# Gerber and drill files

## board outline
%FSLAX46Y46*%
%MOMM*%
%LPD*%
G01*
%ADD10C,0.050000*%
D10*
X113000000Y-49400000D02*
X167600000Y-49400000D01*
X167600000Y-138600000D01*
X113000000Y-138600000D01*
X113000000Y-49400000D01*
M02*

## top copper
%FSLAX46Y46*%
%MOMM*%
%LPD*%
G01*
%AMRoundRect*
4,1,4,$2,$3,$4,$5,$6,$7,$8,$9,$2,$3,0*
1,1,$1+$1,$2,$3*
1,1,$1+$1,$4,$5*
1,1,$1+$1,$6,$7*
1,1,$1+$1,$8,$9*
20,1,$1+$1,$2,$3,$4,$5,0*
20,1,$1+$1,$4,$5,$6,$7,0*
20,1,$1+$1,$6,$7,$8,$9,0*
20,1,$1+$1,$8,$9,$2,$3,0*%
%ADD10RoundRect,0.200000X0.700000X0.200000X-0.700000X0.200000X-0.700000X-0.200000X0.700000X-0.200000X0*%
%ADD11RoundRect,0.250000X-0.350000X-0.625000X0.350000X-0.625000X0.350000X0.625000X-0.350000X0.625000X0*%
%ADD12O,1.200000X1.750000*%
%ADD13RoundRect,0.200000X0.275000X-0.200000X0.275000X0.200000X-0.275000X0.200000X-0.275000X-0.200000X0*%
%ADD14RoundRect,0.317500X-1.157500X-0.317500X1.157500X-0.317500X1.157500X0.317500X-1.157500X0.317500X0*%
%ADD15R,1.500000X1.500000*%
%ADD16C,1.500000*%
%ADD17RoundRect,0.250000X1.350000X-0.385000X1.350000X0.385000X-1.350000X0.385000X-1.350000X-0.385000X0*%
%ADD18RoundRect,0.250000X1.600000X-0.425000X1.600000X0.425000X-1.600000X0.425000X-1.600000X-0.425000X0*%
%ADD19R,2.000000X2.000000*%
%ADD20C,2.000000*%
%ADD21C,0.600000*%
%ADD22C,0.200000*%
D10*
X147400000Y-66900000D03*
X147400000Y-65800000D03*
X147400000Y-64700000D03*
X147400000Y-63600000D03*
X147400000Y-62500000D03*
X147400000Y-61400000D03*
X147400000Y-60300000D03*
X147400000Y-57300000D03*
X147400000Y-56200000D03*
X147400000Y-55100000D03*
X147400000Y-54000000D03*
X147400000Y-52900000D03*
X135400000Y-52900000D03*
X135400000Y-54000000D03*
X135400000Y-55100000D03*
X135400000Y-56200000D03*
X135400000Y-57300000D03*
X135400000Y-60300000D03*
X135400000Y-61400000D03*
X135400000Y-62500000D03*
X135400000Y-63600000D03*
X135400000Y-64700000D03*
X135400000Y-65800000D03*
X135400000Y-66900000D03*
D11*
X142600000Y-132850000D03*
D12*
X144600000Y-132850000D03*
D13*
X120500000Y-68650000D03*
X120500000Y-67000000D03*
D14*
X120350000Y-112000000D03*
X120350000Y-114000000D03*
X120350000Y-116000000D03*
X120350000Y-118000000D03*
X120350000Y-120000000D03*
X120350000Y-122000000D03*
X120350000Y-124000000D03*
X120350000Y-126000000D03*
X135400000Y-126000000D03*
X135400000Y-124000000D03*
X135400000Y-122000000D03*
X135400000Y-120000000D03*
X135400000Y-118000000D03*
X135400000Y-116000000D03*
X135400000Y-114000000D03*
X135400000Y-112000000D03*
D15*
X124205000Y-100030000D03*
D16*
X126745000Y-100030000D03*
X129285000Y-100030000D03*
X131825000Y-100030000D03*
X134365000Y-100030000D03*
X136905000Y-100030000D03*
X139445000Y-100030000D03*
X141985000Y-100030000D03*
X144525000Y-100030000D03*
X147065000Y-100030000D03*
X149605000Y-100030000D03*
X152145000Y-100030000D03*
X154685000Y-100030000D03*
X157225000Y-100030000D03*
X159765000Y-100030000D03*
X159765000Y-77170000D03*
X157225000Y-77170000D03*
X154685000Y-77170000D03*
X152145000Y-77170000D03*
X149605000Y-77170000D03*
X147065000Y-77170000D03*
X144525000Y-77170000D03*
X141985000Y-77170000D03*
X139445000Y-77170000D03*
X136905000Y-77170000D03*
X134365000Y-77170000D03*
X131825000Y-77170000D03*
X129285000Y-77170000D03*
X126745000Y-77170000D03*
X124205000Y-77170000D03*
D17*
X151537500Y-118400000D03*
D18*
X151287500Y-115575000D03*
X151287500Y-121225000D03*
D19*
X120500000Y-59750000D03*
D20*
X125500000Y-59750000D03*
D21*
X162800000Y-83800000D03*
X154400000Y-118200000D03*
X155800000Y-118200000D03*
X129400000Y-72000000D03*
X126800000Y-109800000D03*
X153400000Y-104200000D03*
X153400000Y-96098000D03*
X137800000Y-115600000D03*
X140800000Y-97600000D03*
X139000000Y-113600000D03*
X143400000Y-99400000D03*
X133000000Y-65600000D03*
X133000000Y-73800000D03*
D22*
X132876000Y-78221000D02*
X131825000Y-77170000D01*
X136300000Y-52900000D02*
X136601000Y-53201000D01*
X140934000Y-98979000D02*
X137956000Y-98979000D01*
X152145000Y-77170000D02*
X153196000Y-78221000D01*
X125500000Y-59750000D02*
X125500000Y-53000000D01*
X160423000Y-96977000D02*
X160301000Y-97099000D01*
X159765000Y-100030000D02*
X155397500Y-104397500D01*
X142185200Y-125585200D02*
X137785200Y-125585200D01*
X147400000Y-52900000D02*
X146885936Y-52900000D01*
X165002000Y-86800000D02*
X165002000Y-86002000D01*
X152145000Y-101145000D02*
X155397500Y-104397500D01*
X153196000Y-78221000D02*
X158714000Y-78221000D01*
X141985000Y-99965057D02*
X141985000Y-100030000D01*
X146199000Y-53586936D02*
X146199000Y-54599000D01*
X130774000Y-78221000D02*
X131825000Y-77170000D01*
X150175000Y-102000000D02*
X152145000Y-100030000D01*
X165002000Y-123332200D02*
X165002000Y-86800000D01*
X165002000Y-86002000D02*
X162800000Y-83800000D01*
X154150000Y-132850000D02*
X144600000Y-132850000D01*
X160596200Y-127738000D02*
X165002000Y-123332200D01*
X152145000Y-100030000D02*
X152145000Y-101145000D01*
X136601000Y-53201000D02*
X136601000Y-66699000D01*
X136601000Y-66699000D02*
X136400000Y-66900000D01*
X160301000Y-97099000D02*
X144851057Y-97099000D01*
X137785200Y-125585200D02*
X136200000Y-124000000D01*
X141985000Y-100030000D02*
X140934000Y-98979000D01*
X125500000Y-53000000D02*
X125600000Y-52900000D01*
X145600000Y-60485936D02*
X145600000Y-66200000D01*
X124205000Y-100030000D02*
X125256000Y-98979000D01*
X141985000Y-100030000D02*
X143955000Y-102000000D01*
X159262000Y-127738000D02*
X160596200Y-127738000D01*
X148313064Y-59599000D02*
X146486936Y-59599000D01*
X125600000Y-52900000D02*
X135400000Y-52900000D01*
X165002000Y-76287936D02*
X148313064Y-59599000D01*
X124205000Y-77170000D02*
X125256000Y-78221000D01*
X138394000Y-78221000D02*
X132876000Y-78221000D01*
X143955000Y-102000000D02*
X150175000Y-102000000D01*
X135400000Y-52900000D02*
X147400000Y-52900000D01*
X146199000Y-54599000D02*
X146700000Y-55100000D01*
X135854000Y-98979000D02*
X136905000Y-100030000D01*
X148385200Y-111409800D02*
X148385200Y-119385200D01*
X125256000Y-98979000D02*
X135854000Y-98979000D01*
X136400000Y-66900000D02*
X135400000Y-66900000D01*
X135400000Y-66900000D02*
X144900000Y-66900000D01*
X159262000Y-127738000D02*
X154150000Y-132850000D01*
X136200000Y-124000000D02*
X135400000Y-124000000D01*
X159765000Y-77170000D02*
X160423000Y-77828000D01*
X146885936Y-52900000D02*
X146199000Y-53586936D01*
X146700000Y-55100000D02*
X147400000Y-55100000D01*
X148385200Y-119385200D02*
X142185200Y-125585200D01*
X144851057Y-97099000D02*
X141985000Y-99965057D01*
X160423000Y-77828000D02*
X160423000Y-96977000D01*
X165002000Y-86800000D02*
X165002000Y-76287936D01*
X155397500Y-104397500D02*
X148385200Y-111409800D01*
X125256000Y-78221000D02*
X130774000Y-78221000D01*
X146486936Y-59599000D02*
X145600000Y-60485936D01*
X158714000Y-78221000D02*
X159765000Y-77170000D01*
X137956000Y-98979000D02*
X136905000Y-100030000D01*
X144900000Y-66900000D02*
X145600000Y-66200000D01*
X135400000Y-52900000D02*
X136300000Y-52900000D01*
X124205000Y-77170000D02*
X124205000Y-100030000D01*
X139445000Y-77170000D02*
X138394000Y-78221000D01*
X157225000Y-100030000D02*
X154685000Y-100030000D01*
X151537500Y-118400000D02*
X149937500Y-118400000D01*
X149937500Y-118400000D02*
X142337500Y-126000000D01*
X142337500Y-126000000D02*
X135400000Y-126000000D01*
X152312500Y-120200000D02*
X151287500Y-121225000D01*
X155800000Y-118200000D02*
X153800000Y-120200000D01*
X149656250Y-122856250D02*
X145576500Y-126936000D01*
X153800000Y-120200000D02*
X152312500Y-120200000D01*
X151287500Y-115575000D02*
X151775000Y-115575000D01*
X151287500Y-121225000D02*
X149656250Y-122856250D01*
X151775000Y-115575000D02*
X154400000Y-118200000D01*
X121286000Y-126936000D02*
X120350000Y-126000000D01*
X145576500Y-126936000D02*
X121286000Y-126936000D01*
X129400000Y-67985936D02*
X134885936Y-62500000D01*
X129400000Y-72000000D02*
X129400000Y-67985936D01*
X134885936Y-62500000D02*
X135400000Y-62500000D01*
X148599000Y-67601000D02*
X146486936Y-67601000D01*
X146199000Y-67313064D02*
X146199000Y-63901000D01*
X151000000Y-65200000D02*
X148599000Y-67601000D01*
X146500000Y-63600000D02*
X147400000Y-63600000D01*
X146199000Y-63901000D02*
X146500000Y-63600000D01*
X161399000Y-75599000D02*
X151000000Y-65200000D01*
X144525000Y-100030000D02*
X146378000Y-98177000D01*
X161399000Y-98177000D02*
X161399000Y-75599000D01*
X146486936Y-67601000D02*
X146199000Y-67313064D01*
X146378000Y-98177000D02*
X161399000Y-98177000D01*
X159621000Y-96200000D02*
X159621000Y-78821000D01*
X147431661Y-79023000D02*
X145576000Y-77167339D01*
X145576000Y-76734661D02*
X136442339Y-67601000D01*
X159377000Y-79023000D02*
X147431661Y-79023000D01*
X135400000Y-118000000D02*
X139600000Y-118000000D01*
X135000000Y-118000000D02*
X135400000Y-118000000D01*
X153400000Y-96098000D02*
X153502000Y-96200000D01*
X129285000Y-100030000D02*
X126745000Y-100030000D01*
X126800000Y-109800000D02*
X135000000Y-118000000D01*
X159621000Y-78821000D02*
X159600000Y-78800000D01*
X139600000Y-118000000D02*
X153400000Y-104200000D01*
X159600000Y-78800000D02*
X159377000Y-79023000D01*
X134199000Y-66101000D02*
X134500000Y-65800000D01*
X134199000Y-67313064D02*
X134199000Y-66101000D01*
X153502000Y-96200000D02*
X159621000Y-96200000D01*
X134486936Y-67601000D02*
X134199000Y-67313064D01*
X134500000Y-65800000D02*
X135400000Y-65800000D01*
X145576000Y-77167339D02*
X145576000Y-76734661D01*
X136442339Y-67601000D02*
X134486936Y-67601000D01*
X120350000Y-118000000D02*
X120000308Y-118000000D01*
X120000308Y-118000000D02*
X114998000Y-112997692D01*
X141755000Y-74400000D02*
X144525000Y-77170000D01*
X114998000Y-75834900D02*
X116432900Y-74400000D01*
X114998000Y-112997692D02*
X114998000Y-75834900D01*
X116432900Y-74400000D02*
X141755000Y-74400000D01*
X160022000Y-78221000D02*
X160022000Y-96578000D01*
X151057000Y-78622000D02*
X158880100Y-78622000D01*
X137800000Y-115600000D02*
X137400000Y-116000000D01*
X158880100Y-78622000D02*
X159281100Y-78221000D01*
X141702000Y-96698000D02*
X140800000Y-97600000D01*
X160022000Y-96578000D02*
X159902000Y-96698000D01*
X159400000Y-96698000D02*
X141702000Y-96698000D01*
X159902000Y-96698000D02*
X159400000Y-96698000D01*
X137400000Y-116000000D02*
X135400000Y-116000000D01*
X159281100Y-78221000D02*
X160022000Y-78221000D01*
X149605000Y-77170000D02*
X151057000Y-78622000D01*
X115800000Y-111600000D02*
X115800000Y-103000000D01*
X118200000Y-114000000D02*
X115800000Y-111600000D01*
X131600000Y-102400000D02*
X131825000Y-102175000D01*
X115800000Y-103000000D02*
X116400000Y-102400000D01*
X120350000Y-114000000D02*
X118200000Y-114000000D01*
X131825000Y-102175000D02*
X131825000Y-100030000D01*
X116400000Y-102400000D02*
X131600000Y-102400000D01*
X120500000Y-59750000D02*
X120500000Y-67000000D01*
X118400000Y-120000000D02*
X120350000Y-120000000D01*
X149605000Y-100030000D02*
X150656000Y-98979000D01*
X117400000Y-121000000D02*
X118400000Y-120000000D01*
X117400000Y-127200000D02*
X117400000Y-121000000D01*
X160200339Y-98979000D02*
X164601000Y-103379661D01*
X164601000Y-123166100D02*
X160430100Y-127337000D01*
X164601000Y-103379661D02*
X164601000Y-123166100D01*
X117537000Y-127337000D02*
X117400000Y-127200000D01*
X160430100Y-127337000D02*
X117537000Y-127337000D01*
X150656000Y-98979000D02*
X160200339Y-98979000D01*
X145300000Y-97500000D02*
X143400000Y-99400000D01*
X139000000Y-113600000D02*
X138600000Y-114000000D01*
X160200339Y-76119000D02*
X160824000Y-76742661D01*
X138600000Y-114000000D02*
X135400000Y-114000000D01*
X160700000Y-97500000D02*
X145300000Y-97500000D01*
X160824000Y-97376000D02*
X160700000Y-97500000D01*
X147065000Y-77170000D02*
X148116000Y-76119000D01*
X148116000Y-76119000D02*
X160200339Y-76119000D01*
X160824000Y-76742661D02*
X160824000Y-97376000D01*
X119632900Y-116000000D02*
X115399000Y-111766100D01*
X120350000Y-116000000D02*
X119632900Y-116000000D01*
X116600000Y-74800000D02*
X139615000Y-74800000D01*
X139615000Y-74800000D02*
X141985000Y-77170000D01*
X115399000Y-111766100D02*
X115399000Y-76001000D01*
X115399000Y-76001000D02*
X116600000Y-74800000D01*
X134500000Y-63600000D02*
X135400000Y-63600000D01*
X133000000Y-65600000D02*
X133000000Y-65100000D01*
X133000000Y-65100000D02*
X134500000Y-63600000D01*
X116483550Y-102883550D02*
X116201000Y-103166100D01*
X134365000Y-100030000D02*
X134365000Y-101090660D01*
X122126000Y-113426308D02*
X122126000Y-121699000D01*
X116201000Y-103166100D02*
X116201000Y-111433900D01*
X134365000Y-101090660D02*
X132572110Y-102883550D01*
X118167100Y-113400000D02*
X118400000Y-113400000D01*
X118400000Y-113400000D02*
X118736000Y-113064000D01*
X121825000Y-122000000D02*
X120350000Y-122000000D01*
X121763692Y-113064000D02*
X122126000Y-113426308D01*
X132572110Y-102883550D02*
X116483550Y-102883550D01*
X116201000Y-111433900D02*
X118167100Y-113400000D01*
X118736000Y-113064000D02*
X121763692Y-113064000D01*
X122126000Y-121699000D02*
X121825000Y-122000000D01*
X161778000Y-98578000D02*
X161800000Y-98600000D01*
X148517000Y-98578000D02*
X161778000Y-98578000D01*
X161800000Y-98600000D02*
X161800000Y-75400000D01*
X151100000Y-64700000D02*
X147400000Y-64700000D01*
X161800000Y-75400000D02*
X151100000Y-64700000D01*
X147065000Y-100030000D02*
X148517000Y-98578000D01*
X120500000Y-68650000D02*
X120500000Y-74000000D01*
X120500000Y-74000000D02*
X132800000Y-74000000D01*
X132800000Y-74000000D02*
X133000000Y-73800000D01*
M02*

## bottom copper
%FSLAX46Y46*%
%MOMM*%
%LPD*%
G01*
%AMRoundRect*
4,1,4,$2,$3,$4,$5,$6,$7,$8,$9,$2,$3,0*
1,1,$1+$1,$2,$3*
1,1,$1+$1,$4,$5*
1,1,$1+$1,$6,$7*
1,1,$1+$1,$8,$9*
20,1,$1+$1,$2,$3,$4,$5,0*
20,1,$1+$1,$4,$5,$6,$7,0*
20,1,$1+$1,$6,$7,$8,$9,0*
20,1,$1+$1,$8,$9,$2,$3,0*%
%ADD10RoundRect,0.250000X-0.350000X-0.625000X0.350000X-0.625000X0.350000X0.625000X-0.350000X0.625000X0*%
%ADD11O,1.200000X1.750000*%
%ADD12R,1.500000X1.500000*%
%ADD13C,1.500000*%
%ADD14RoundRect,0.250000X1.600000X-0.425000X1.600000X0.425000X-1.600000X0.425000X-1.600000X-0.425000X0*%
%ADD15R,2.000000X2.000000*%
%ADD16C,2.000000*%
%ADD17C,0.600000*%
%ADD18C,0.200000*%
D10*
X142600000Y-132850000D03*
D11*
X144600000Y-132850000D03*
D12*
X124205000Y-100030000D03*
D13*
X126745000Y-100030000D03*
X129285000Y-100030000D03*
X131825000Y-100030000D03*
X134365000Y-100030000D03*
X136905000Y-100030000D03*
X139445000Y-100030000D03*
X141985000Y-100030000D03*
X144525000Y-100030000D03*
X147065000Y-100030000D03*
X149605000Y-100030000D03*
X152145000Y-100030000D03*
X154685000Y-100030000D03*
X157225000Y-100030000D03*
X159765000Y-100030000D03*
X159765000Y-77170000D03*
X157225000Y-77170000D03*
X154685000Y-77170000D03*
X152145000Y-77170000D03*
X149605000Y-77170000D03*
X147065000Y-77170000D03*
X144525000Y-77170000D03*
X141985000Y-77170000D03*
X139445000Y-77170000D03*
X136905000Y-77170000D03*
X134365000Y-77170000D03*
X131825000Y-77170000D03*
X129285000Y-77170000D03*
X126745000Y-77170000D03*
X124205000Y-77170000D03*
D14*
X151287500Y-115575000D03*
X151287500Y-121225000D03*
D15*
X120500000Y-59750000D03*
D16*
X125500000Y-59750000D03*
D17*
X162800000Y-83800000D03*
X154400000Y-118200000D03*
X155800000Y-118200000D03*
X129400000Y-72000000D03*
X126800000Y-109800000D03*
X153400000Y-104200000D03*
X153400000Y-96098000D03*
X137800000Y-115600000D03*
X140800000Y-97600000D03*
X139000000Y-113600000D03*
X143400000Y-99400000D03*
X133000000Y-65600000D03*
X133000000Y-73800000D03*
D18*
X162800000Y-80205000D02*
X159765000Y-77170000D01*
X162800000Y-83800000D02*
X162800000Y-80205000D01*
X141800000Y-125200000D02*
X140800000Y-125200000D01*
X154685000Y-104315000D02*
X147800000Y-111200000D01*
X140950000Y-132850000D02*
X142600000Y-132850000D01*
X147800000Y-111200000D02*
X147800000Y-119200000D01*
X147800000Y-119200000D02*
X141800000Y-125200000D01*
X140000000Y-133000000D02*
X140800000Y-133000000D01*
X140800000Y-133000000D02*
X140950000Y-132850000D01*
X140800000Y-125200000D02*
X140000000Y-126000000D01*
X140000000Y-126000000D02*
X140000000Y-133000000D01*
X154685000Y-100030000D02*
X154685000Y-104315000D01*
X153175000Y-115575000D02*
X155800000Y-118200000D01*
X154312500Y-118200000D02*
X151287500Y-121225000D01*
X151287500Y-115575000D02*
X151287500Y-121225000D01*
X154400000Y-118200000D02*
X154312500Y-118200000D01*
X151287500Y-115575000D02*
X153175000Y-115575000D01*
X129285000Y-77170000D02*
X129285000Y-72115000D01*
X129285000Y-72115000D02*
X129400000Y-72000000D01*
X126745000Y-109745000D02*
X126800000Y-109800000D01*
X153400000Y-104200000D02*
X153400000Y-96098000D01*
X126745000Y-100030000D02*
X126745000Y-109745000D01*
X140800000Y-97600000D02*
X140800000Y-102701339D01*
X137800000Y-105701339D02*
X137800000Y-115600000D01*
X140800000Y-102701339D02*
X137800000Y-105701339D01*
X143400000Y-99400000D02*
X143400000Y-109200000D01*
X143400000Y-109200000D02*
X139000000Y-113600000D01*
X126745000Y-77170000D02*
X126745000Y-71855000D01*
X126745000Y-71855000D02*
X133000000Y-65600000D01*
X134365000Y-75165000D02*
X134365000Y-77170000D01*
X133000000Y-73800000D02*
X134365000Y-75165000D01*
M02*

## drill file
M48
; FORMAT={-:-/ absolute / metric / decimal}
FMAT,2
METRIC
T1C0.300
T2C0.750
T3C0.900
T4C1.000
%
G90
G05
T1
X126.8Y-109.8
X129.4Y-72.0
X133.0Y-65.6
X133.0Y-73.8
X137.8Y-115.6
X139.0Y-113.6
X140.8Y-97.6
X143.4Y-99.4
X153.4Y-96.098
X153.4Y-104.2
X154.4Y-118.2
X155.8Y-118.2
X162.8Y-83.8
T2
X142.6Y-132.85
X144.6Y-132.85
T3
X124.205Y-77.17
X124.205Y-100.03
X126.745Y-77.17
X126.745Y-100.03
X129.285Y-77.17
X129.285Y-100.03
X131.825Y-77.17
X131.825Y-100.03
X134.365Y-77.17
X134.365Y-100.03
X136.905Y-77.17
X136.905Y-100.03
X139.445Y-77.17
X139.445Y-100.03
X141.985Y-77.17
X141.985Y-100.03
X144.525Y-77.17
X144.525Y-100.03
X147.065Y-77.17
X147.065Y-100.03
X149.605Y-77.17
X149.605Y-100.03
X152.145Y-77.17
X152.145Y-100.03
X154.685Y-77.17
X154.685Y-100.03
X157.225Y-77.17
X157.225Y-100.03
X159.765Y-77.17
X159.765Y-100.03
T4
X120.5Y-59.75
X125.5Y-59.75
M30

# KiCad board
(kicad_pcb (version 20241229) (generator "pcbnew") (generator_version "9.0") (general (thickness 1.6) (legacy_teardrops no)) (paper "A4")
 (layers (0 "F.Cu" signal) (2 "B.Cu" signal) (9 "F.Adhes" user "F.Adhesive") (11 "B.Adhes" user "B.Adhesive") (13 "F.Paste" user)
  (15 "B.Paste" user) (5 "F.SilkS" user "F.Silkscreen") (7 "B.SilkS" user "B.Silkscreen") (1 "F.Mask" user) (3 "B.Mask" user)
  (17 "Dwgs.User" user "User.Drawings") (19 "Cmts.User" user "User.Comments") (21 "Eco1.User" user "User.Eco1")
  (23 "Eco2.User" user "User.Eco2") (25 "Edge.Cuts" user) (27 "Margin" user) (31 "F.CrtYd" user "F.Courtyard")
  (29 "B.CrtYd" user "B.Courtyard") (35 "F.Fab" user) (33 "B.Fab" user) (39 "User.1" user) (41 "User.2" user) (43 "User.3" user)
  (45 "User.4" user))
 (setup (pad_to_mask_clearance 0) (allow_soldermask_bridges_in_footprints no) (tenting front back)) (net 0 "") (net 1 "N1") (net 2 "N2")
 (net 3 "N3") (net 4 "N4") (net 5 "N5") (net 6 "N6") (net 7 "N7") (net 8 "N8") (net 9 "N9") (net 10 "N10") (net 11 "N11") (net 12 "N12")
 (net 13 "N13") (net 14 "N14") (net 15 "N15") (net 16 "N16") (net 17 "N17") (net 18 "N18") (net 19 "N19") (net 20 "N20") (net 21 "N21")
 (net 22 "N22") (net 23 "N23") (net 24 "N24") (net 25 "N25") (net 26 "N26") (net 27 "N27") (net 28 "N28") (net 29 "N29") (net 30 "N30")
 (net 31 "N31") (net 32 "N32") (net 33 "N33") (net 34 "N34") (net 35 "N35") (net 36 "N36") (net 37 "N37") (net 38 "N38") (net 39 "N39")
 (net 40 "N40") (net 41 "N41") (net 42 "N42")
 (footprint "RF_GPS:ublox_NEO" (layer "F.Cu") (at 141.4 59.9 180)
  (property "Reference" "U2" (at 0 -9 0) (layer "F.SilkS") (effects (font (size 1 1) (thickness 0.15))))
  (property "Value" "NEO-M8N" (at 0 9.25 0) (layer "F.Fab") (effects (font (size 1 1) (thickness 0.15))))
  (pad "1" smd roundrect (at -6 -7 180) (size 1.8 0.8) (layers "F.Cu" "F.Mask" "F.Paste") (roundrect_rratio 0.25) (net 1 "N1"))
  (pad "2" smd roundrect (at -6 -5.9 180) (size 1.8 0.8) (layers "F.Cu" "F.Mask" "F.Paste") (roundrect_rratio 0.25) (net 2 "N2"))
  (pad "3" smd roundrect (at -6 -4.8 180) (size 1.8 0.8) (layers "F.Cu" "F.Mask" "F.Paste") (roundrect_rratio 0.25) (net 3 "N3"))
  (pad "4" smd roundrect (at -6 -3.7 180) (size 1.8 0.8) (layers "F.Cu" "F.Mask" "F.Paste") (roundrect_rratio 0.25) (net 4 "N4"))
  (pad "5" smd roundrect (at -6 -2.6 180) (size 1.8 0.8) (layers "F.Cu" "F.Mask" "F.Paste") (roundrect_rratio 0.25) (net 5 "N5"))
  (pad "6" smd roundrect (at -6 -1.5 180) (size 1.8 0.8) (layers "F.Cu" "F.Mask" "F.Paste") (roundrect_rratio 0.25) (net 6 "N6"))
  (pad "7" smd roundrect (at -6 -0.4 180) (size 1.8 0.8) (layers "F.Cu" "F.Mask" "F.Paste") (roundrect_rratio 0.25) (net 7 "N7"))
  (pad "8" smd roundrect (at -6 2.6 180) (size 1.8 0.8) (layers "F.Cu" "F.Mask" "F.Paste") (roundrect_rratio 0.25) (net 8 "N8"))
  (pad "9" smd roundrect (at -6 3.7 180) (size 1.8 0.8) (layers "F.Cu" "F.Mask" "F.Paste") (roundrect_rratio 0.25) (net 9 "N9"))
  (pad "10" smd roundrect (at -6 4.8 180) (size 1.8 0.8) (layers "F.Cu" "F.Mask" "F.Paste") (roundrect_rratio 0.25) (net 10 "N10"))
  (pad "11" smd roundrect (at -6 5.9 180) (size 1.8 0.8) (layers "F.Cu" "F.Mask" "F.Paste") (roundrect_rratio 0.25) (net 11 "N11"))
  (pad "12" smd roundrect (at -6 7 180) (size 1.8 0.8) (layers "F.Cu" "F.Mask" "F.Paste") (roundrect_rratio 0.25) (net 10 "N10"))
  (pad "13" smd roundrect (at 6 7 180) (size 1.8 0.8) (layers "F.Cu" "F.Mask" "F.Paste") (roundrect_rratio 0.25) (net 10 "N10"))
  (pad "14" smd roundrect (at 6 5.9 180) (size 1.8 0.8) (layers "F.Cu" "F.Mask" "F.Paste") (roundrect_rratio 0.25) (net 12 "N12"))
  (pad "15" smd roundrect (at 6 4.8 180) (size 1.8 0.8) (layers "F.Cu" "F.Mask" "F.Paste") (roundrect_rratio 0.25) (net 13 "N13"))
  (pad "16" smd roundrect (at 6 3.7 180) (size 1.8 0.8) (layers "F.Cu" "F.Mask" "F.Paste") (roundrect_rratio 0.25) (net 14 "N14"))
  (pad "17" smd roundrect (at 6 2.6 180) (size 1.8 0.8) (layers "F.Cu" "F.Mask" "F.Paste") (roundrect_rratio 0.25) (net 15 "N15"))
  (pad "18" smd roundrect (at 6 -0.4 180) (size 1.8 0.8) (layers "F.Cu" "F.Mask" "F.Paste") (roundrect_rratio 0.25) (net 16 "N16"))
  (pad "19" smd roundrect (at 6 -1.5 180) (size 1.8 0.8) (layers "F.Cu" "F.Mask" "F.Paste") (roundrect_rratio 0.25) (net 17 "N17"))
  (pad "20" smd roundrect (at 6 -2.6 180) (size 1.8 0.8) (layers "F.Cu" "F.Mask" "F.Paste") (roundrect_rratio 0.25) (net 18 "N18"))
  (pad "21" smd roundrect (at 6 -3.7 180) (size 1.8 0.8) (layers "F.Cu" "F.Mask" "F.Paste") (roundrect_rratio 0.25) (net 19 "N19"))
  (pad "22" smd roundrect (at 6 -4.8 180) (size 1.8 0.8) (layers "F.Cu" "F.Mask" "F.Paste") (roundrect_rratio 0.25) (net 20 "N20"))
  (pad "23" smd roundrect (at 6 -5.9 180) (size 1.8 0.8) (layers "F.Cu" "F.Mask" "F.Paste") (roundrect_rratio 0.25) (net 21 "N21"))
  (pad "24" smd roundrect (at 6 -7 180) (size 1.8 0.8) (layers "F.Cu" "F.Mask" "F.Paste") (roundrect_rratio 0.25) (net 10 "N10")))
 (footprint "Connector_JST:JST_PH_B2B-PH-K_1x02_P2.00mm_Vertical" (layer "F.Cu") (at 142.6 132.85)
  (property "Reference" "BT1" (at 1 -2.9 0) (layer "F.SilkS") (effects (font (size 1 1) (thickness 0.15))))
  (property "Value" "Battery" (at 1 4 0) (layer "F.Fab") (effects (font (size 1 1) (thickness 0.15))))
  (pad "1" thru_hole roundrect (at 0 0) (size 1.2 1.75) (drill 0.75) (layers "*.Cu" "*.Mask") (remove_unused_layers no)
   (roundrect_rratio 0.208333) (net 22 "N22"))
  (pad "2" thru_hole oval (at 2 0) (size 1.2 1.75) (drill 0.75) (layers "*.Cu" "*.Mask") (remove_unused_layers no) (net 10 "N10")))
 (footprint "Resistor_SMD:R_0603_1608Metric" (layer "F.Cu") (at 120.5 67.825 90)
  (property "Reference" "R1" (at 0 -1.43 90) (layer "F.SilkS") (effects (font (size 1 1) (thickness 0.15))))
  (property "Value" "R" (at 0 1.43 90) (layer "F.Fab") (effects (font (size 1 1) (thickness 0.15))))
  (pad "1" smd roundrect (at -0.825 0 90) (size 0.8 0.95) (layers "F.Cu" "F.Mask" "F.Paste") (roundrect_rratio 0.25) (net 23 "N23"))
  (pad "2" smd roundrect (at 0.825 0 90) (size 0.8 0.95) (layers "F.Cu" "F.Mask" "F.Paste") (roundrect_rratio 0.25) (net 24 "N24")))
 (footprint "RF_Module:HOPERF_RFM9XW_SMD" (layer "F.Cu") (at 127.875 119)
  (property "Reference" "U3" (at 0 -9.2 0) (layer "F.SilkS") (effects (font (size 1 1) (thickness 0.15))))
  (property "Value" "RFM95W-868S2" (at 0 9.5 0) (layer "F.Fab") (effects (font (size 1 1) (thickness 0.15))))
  (pad "1" smd roundrect (at -7.525 -7) (size 2.95 1.27) (layers "F.Cu" "F.Mask" "F.Paste") (roundrect_rratio 0.25) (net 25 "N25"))
  (pad "2" smd roundrect (at -7.525 -5) (size 2.95 1.27) (layers "F.Cu" "F.Mask" "F.Paste") (roundrect_rratio 0.25) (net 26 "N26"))
  (pad "3" smd roundrect (at -7.525 -3) (size 2.95 1.27) (layers "F.Cu" "F.Mask" "F.Paste") (roundrect_rratio 0.25) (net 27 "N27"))
  (pad "4" smd roundrect (at -7.525 -1) (size 2.95 1.27) (layers "F.Cu" "F.Mask" "F.Paste") (roundrect_rratio 0.25) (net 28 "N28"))
  (pad "5" smd roundrect (at -7.525 1) (size 2.95 1.27) (layers "F.Cu" "F.Mask" "F.Paste") (roundrect_rratio 0.25) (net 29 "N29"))
  (pad "6" smd roundrect (at -7.525 3) (size 2.95 1.27) (layers "F.Cu" "F.Mask" "F.Paste") (roundrect_rratio 0.25) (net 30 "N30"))
  (pad "7" smd roundrect (at -7.525 5) (size 2.95 1.27) (layers "F.Cu" "F.Mask" "F.Paste") (roundrect_rratio 0.25) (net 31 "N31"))
  (pad "8" smd roundrect (at -7.525 7) (size 2.95 1.27) (layers "F.Cu" "F.Mask" "F.Paste") (roundrect_rratio 0.25) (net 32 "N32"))
  (pad "9" smd roundrect (at 7.525 7) (size 2.95 1.27) (layers "F.Cu" "F.Mask" "F.Paste") (roundrect_rratio 0.25) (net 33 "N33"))
  (pad "10" smd roundrect (at 7.525 5) (size 2.95 1.27) (layers "F.Cu" "F.Mask" "F.Paste") (roundrect_rratio 0.25) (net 10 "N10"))
  (pad "11" smd roundrect (at 7.525 3) (size 2.95 1.27) (layers "F.Cu" "F.Mask" "F.Paste") (roundrect_rratio 0.25) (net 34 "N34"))
  (pad "12" smd roundrect (at 7.525 1) (size 2.95 1.27) (layers "F.Cu" "F.Mask" "F.Paste") (roundrect_rratio 0.25) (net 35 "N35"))
  (pad "13" smd roundrect (at 7.525 -1) (size 2.95 1.27) (layers "F.Cu" "F.Mask" "F.Paste") (roundrect_rratio 0.25) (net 21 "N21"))
  (pad "14" smd roundrect (at 7.525 -3) (size 2.95 1.27) (layers "F.Cu" "F.Mask" "F.Paste") (roundrect_rratio 0.25) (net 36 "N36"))
  (pad "15" smd roundrect (at 7.525 -5) (size 2.95 1.27) (layers "F.Cu" "F.Mask" "F.Paste") (roundrect_rratio 0.25) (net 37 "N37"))
  (pad "16" smd roundrect (at 7.525 -7) (size 2.95 1.27) (layers "F.Cu" "F.Mask" "F.Paste") (roundrect_rratio 0.25) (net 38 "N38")))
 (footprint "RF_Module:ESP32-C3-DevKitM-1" (layer "F.Cu") (at 124.205 100.03 90)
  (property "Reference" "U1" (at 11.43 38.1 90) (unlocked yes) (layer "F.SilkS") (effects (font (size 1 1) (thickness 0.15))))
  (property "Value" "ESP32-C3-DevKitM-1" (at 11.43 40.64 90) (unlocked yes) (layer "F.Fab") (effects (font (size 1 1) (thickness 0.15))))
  (pad "1" thru_hole rect (at 0 0 90) (size 1.5 1.5) (drill 0.9) (layers "*.Cu" "*.Mask") (remove_unused_layers yes) (keep_end_layers yes)
   (zone_layer_connections) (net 10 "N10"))
  (pad "2" thru_hole circle (at 0 2.54 90) (size 1.5 1.5) (drill 0.9) (layers "*.Cu" "*.Mask") (remove_unused_layers yes)
   (keep_end_layers yes) (zone_layer_connections) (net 21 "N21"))
  (pad "3" thru_hole circle (at 0 5.08 90) (size 1.5 1.5) (drill 0.9) (layers "*.Cu" "*.Mask") (remove_unused_layers yes)
   (keep_end_layers yes) (zone_layer_connections) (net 21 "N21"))
  (pad "4" thru_hole circle (at 0 7.62 90) (size 1.5 1.5) (drill 0.9) (layers "*.Cu" "*.Mask") (remove_unused_layers yes)
   (keep_end_layers yes) (zone_layer_connections) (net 26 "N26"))
  (pad "5" thru_hole circle (at 0 10.16 90) (size 1.5 1.5) (drill 0.9) (layers "*.Cu" "*.Mask") (remove_unused_layers yes)
   (keep_end_layers yes) (zone_layer_connections) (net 30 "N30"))
  (pad "6" thru_hole circle (at 0 12.7 90) (size 1.5 1.5) (drill 0.9) (layers "*.Cu" "*.Mask") (remove_unused_layers yes)
   (keep_end_layers yes) (zone_layer_connections) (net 10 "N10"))
  (pad "7" thru_hole circle (at 0 15.24 90) (size 1.5 1.5) (drill 0.9) (layers "*.Cu" "*.Mask") (remove_unused_layers yes)
   (keep_end_layers yes) (zone_layer_connections) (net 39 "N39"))
  (pad "8" thru_hole circle (at 0 17.78 90) (size 1.5 1.5) (drill 0.9) (layers "*.Cu" "*.Mask") (remove_unused_layers yes)
   (keep_end_layers yes) (zone_layer_connections) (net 10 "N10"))
  (pad "9" thru_hole circle (at 0 20.32 90) (size 1.5 1.5) (drill 0.9) (layers "*.Cu" "*.Mask") (remove_unused_layers yes)
   (keep_end_layers yes) (zone_layer_connections) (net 4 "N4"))
  (pad "10" thru_hole circle (at 0 22.86 90) (size 1.5 1.5) (drill 0.9) (layers "*.Cu" "*.Mask") (remove_unused_layers yes)
   (keep_end_layers yes) (zone_layer_connections) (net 3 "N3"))
  (pad "11" thru_hole circle (at 0 25.4 90) (size 1.5 1.5) (drill 0.9) (layers "*.Cu" "*.Mask") (remove_unused_layers yes)
   (keep_end_layers yes) (zone_layer_connections) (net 29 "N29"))
  (pad "12" thru_hole circle (at 0 27.94 90) (size 1.5 1.5) (drill 0.9) (layers "*.Cu" "*.Mask") (remove_unused_layers yes)
   (keep_end_layers yes) (zone_layer_connections) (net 10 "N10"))
  (pad "13" thru_hole circle (at 0 30.48 90) (size 1.5 1.5) (drill 0.9) (layers "*.Cu" "*.Mask") (remove_unused_layers yes)
   (keep_end_layers yes) (zone_layer_connections) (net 22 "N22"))
  (pad "14" thru_hole circle (at 0 33.02 90) (size 1.5 1.5) (drill 0.9) (layers "*.Cu" "*.Mask") (remove_unused_layers yes)
   (keep_end_layers yes) (zone_layer_connections) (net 22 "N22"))
  (pad "15" thru_hole circle (at 0 35.56 90) (size 1.5 1.5) (drill 0.9) (layers "*.Cu" "*.Mask") (remove_unused_layers yes)
   (keep_end_layers yes) (zone_layer_connections) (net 10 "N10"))
  (pad "16" thru_hole circle (at 22.86 35.56 90) (size 1.5 1.5) (drill 0.9) (layers "*.Cu" "*.Mask") (remove_unused_layers yes)
   (keep_end_layers yes) (zone_layer_connections) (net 10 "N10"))
  (pad "17" thru_hole circle (at 22.86 33.02 90) (size 1.5 1.5) (drill 0.9) (layers "*.Cu" "*.Mask") (remove_unused_layers yes)
   (keep_end_layers yes) (zone_layer_connections) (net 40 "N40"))
  (pad "18" thru_hole circle (at 22.86 30.48 90) (size 1.5 1.5) (drill 0.9) (layers "*.Cu" "*.Mask") (remove_unused_layers yes)
   (keep_end_layers yes) (zone_layer_connections) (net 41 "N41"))
  (pad "19" thru_hole circle (at 22.86 27.94 90) (size 1.5 1.5) (drill 0.9) (layers "*.Cu" "*.Mask") (remove_unused_layers yes)
   (keep_end_layers yes) (zone_layer_connections) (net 10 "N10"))
  (pad "20" thru_hole circle (at 22.86 25.4 90) (size 1.5 1.5) (drill 0.9) (layers "*.Cu" "*.Mask") (remove_unused_layers yes)
   (keep_end_layers yes) (zone_layer_connections) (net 36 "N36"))
  (pad "21" thru_hole circle (at 22.86 22.86 90) (size 1.5 1.5) (drill 0.9) (layers "*.Cu" "*.Mask") (remove_unused_layers yes)
   (keep_end_layers yes) (zone_layer_connections) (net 37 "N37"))
  (pad "22" thru_hole circle (at 22.86 20.32 90) (size 1.5 1.5) (drill 0.9) (layers "*.Cu" "*.Mask") (remove_unused_layers yes)
   (keep_end_layers yes) (zone_layer_connections) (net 28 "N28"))
  (pad "23" thru_hole circle (at 22.86 17.78 90) (size 1.5 1.5) (drill 0.9) (layers "*.Cu" "*.Mask") (remove_unused_layers yes)
   (keep_end_layers yes) (zone_layer_connections) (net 27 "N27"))
  (pad "24" thru_hole circle (at 22.86 15.24 90) (size 1.5 1.5) (drill 0.9) (layers "*.Cu" "*.Mask") (remove_unused_layers yes)
   (keep_end_layers yes) (zone_layer_connections) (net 10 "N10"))
  (pad "25" thru_hole circle (at 22.86 12.7 90) (size 1.5 1.5) (drill 0.9) (layers "*.Cu" "*.Mask") (remove_unused_layers yes)
   (keep_end_layers yes) (zone_layer_connections) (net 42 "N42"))
  (pad "26" thru_hole circle (at 22.86 10.16 90) (size 1.5 1.5) (drill 0.9) (layers "*.Cu" "*.Mask") (remove_unused_layers yes)
   (keep_end_layers yes) (zone_layer_connections) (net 23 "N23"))
  (pad "27" thru_hole circle (at 22.86 7.62 90) (size 1.5 1.5) (drill 0.9) (layers "*.Cu" "*.Mask") (remove_unused_layers yes)
   (keep_end_layers yes) (zone_layer_connections) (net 10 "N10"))
  (pad "28" thru_hole circle (at 22.86 5.08 90) (size 1.5 1.5) (drill 0.9) (layers "*.Cu" "*.Mask") (remove_unused_layers yes)
   (keep_end_layers yes) (zone_layer_connections) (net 18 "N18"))
  (pad "29" thru_hole circle (at 22.86 2.54 90) (size 1.5 1.5) (drill 0.9) (layers "*.Cu" "*.Mask") (remove_unused_layers yes)
   (keep_end_layers yes) (zone_layer_connections) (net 19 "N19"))
  (pad "30" thru_hole circle (at 22.86 0 90) (size 1.5 1.5) (drill 0.9) (layers "*.Cu" "*.Mask") (remove_unused_layers yes)
   (keep_end_layers yes) (zone_layer_connections) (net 10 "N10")))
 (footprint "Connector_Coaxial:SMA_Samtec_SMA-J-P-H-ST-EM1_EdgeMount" (layer "F.Cu") (at 151.5375 118.4)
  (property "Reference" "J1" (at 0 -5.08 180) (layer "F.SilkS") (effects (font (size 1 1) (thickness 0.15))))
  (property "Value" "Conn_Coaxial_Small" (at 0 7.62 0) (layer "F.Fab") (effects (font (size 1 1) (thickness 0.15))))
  (pad "1" smd roundrect (at 0 0 90) (size 1.27 3.2) (layers "F.Cu" "F.Mask") (roundrect_rratio 0.1968503937) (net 33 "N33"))
  (pad "2" smd roundrect (at -0.25 -2.825 90) (size 1.35 3.7) (layers "F.Cu" "F.Mask") (roundrect_rratio 0.1851851852) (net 32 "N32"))
  (pad "2" smd roundrect (at -0.25 -2.825 90) (size 1.35 3.7) (layers "B.Cu" "B.Mask") (roundrect_rratio 0.1851851852) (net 32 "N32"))
  (pad "2" smd roundrect (at -0.25 2.825 90) (size 1.35 3.7) (layers "F.Cu" "F.Mask") (roundrect_rratio 0.1851851852) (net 32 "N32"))
  (pad "2" smd roundrect (at -0.25 2.825 90) (size 1.35 3.7) (layers "B.Cu" "B.Mask") (roundrect_rratio 0.1851851852) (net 32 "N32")))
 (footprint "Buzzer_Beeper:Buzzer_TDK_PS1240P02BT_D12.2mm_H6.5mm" (layer "F.Cu") (at 120.5 59.75)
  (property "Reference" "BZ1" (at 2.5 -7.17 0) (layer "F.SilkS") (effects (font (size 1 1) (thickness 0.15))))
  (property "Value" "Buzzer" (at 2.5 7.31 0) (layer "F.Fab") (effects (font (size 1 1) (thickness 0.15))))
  (pad "1" thru_hole rect (at 0 0) (size 2 2) (drill 1) (layers "*.Cu" "*.Mask") (remove_unused_layers no) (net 24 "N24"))
  (pad "2" thru_hole circle (at 5 0) (size 2 2) (drill 1) (layers "*.Cu" "*.Mask") (remove_unused_layers no) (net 10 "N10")))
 (gr_rect (start 113 49.4) (end 167.6 138.6) (stroke (width 0.05) (type default)) (fill no) (layer "Edge.Cuts"))
 (segment (start 132.876 78.221) (end 131.825 77.17) (width 0.2) (layer "F.Cu") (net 10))
 (segment (start 136.3 52.9) (end 136.601 53.201) (width 0.2) (layer "F.Cu") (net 10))
 (segment (start 140.934 98.979) (end 137.956 98.979) (width 0.2) (layer "F.Cu") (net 10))
 (segment (start 152.145 77.17) (end 153.196 78.221) (width 0.2) (layer "F.Cu") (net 10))
 (segment (start 125.5 59.75) (end 125.5 53) (width 0.2) (layer "F.Cu") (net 10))
 (segment (start 160.423 96.977) (end 160.301 97.099) (width 0.2) (layer "F.Cu") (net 10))
 (segment (start 159.765 100.03) (end 155.3975 104.3975) (width 0.2) (layer "F.Cu") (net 10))
 (segment (start 142.1852 125.5852) (end 137.7852 125.5852) (width 0.2) (layer "F.Cu") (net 10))
 (segment (start 147.4 52.9) (end 146.885936 52.9) (width 0.2) (layer "F.Cu") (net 10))
 (segment (start 165.002 86.8) (end 165.002 86.002) (width 0.2) (layer "F.Cu") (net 10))
 (segment (start 152.145 101.145) (end 155.3975 104.3975) (width 0.2) (layer "F.Cu") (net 10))
 (segment (start 153.196 78.221) (end 158.714 78.221) (width 0.2) (layer "F.Cu") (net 10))
 (segment (start 141.985 99.965057) (end 141.985 100.03) (width 0.2) (layer "F.Cu") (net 10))
 (segment (start 146.199 53.586936) (end 146.199 54.599) (width 0.2) (layer "F.Cu") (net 10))
 (segment (start 130.774 78.221) (end 131.825 77.17) (width 0.2) (layer "F.Cu") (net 10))
 (segment (start 150.175 102) (end 152.145 100.03) (width 0.2) (layer "F.Cu") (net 10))
 (segment (start 165.002 123.3322) (end 165.002 86.8) (width 0.2) (layer "F.Cu") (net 10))
 (segment (start 165.002 86.002) (end 162.8 83.8) (width 0.2) (layer "F.Cu") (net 10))
 (segment (start 154.15 132.85) (end 144.6 132.85) (width 0.2) (layer "F.Cu") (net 10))
 (segment (start 160.5962 127.738) (end 165.002 123.3322) (width 0.2) (layer "F.Cu") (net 10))
 (segment (start 152.145 100.03) (end 152.145 101.145) (width 0.2) (layer "F.Cu") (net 10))
 (segment (start 136.601 53.201) (end 136.601 66.699) (width 0.2) (layer "F.Cu") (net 10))
 (segment (start 136.601 66.699) (end 136.4 66.9) (width 0.2) (layer "F.Cu") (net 10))
 (segment (start 160.301 97.099) (end 144.851057 97.099) (width 0.2) (layer "F.Cu") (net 10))
 (segment (start 137.7852 125.5852) (end 136.2 124) (width 0.2) (layer "F.Cu") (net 10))
 (segment (start 141.985 100.03) (end 140.934 98.979) (width 0.2) (layer "F.Cu") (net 10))
 (segment (start 125.5 53) (end 125.6 52.9) (width 0.2) (layer "F.Cu") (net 10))
 (segment (start 145.6 60.485936) (end 145.6 66.2) (width 0.2) (layer "F.Cu") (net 10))
 (segment (start 124.205 100.03) (end 125.256 98.979) (width 0.2) (layer "F.Cu") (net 10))
 (segment (start 141.985 100.03) (end 143.955 102) (width 0.2) (layer "F.Cu") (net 10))
 (segment (start 159.262 127.738) (end 160.5962 127.738) (width 0.2) (layer "F.Cu") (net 10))
 (segment (start 148.313064 59.599) (end 146.486936 59.599) (width 0.2) (layer "F.Cu") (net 10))
 (segment (start 125.6 52.9) (end 135.4 52.9) (width 0.2) (layer "F.Cu") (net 10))
 (segment (start 165.002 76.287936) (end 148.313064 59.599) (width 0.2) (layer "F.Cu") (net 10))
 (segment (start 124.205 77.17) (end 125.256 78.221) (width 0.2) (layer "F.Cu") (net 10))
 (segment (start 138.394 78.221) (end 132.876 78.221) (width 0.2) (layer "F.Cu") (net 10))
 (segment (start 143.955 102) (end 150.175 102) (width 0.2) (layer "F.Cu") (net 10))
 (segment (start 135.4 52.9) (end 147.4 52.9) (width 0.2) (layer "F.Cu") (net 10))
 (segment (start 146.199 54.599) (end 146.7 55.1) (width 0.2) (layer "F.Cu") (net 10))
 (segment (start 135.854 98.979) (end 136.905 100.03) (width 0.2) (layer "F.Cu") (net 10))
 (segment (start 148.3852 111.4098) (end 148.3852 119.3852) (width 0.2) (layer "F.Cu") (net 10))
 (segment (start 125.256 98.979) (end 135.854 98.979) (width 0.2) (layer "F.Cu") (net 10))
 (segment (start 136.4 66.9) (end 135.4 66.9) (width 0.2) (layer "F.Cu") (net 10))
 (segment (start 135.4 66.9) (end 144.9 66.9) (width 0.2) (layer "F.Cu") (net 10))
 (segment (start 159.262 127.738) (end 154.15 132.85) (width 0.2) (layer "F.Cu") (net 10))
 (segment (start 136.2 124) (end 135.4 124) (width 0.2) (layer "F.Cu") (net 10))
 (segment (start 159.765 77.17) (end 160.423 77.828) (width 0.2) (layer "F.Cu") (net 10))
 (segment (start 146.885936 52.9) (end 146.199 53.586936) (width 0.2) (layer "F.Cu") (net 10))
 (segment (start 146.7 55.1) (end 147.4 55.1) (width 0.2) (layer "F.Cu") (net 10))
 (segment (start 148.3852 119.3852) (end 142.1852 125.5852) (width 0.2) (layer "F.Cu") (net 10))
 (segment (start 144.851057 97.099) (end 141.985 99.965057) (width 0.2) (layer "F.Cu") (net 10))
 (segment (start 160.423 77.828) (end 160.423 96.977) (width 0.2) (layer "F.Cu") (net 10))
 (segment (start 165.002 86.8) (end 165.002 76.287936) (width 0.2) (layer "F.Cu") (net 10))
 (segment (start 155.3975 104.3975) (end 148.3852 111.4098) (width 0.2) (layer "F.Cu") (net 10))
 (segment (start 125.256 78.221) (end 130.774 78.221) (width 0.2) (layer "F.Cu") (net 10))
 (segment (start 146.486936 59.599) (end 145.6 60.485936) (width 0.2) (layer "F.Cu") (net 10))
 (segment (start 158.714 78.221) (end 159.765 77.17) (width 0.2) (layer "F.Cu") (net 10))
 (segment (start 137.956 98.979) (end 136.905 100.03) (width 0.2) (layer "F.Cu") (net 10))
 (segment (start 144.9 66.9) (end 145.6 66.2) (width 0.2) (layer "F.Cu") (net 10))
 (segment (start 135.4 52.9) (end 136.3 52.9) (width 0.2) (layer "F.Cu") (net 10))
 (segment (start 124.205 77.17) (end 124.205 100.03) (width 0.2) (layer "F.Cu") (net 10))
 (segment (start 139.445 77.17) (end 138.394 78.221) (width 0.2) (layer "F.Cu") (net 10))
 (via (at 162.8 83.8) (size 0.6) (drill 0.3) (layers "F.Cu" "B.Cu") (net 10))
 (segment (start 162.8 80.205) (end 159.765 77.17) (width 0.2) (layer "B.Cu") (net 10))
 (segment (start 162.8 83.8) (end 162.8 80.205) (width 0.2) (layer "B.Cu") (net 10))
 (segment (start 157.225 100.03) (end 154.685 100.03) (width 0.2) (layer "F.Cu") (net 22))
 (segment (start 141.8 125.2) (end 140.8 125.2) (width 0.2) (layer "B.Cu") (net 22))
 (segment (start 154.685 104.315) (end 147.8 111.2) (width 0.2) (layer "B.Cu") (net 22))
 (segment (start 140.95 132.85) (end 142.6 132.85) (width 0.2) (layer "B.Cu") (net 22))
 (segment (start 147.8 111.2) (end 147.8 119.2) (width 0.2) (layer "B.Cu") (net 22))
 (segment (start 147.8 119.2) (end 141.8 125.2) (width 0.2) (layer "B.Cu") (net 22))
 (segment (start 140 133) (end 140.8 133) (width 0.2) (layer "B.Cu") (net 22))
 (segment (start 140.8 133) (end 140.95 132.85) (width 0.2) (layer "B.Cu") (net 22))
 (segment (start 140.8 125.2) (end 140 126) (width 0.2) (layer "B.Cu") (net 22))
 (segment (start 140 126) (end 140 133) (width 0.2) (layer "B.Cu") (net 22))
 (segment (start 154.685 100.03) (end 154.685 104.315) (width 0.2) (layer "B.Cu") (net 22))
 (segment (start 151.5375 118.4) (end 149.9375 118.4) (width 0.2) (layer "F.Cu") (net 33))
 (segment (start 149.9375 118.4) (end 142.3375 126) (width 0.2) (layer "F.Cu") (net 33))
 (segment (start 142.3375 126) (end 135.4 126) (width 0.2) (layer "F.Cu") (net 33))
 (segment (start 152.3125 120.2) (end 151.2875 121.225) (width 0.2) (layer "F.Cu") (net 32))
 (segment (start 155.8 118.2) (end 153.8 120.2) (width 0.2) (layer "F.Cu") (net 32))
 (segment (start 149.65625 122.85625) (end 145.5765 126.936) (width 0.2) (layer "F.Cu") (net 32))
 (segment (start 153.8 120.2) (end 152.3125 120.2) (width 0.2) (layer "F.Cu") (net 32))
 (segment (start 151.2875 115.575) (end 151.775 115.575) (width 0.2) (layer "F.Cu") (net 32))
 (segment (start 151.2875 121.225) (end 149.65625 122.85625) (width 0.2) (layer "F.Cu") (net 32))
 (segment (start 151.775 115.575) (end 154.4 118.2) (width 0.2) (layer "F.Cu") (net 32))
 (segment (start 121.286 126.936) (end 120.35 126) (width 0.2) (layer "F.Cu") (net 32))
 (segment (start 145.5765 126.936) (end 121.286 126.936) (width 0.2) (layer "F.Cu") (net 32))
 (via (at 154.4 118.2) (size 0.6) (drill 0.3) (layers "F.Cu" "B.Cu") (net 32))
 (via (at 155.8 118.2) (size 0.6) (drill 0.3) (layers "F.Cu" "B.Cu") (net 32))
 (segment (start 153.175 115.575) (end 155.8 118.2) (width 0.2) (layer "B.Cu") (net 32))
 (segment (start 154.3125 118.2) (end 151.2875 121.225) (width 0.2) (layer "B.Cu") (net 32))
 (segment (start 151.2875 115.575) (end 151.2875 121.225) (width 0.2) (layer "B.Cu") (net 32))
 (segment (start 154.4 118.2) (end 154.3125 118.2) (width 0.2) (layer "B.Cu") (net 32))
 (segment (start 151.2875 115.575) (end 153.175 115.575) (width 0.2) (layer "B.Cu") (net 32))
 (segment (start 129.4 67.985936) (end 134.885936 62.5) (width 0.2) (layer "F.Cu") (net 18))
 (segment (start 129.4 72) (end 129.4 67.985936) (width 0.2) (layer "F.Cu") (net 18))
 (segment (start 134.885936 62.5) (end 135.4 62.5) (width 0.2) (layer "F.Cu") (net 18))
 (via (at 129.4 72) (size 0.6) (drill 0.3) (layers "F.Cu" "B.Cu") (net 18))
 (segment (start 129.285 77.17) (end 129.285 72.115) (width 0.2) (layer "B.Cu") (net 18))
 (segment (start 129.285 72.115) (end 129.4 72) (width 0.2) (layer "B.Cu") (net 18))
 (segment (start 148.599 67.601) (end 146.486936 67.601) (width 0.2) (layer "F.Cu") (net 4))
 (segment (start 146.199 67.313064) (end 146.199 63.901) (width 0.2) (layer "F.Cu") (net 4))
 (segment (start 151 65.2) (end 148.599 67.601) (width 0.2) (layer "F.Cu") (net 4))
 (segment (start 146.5 63.6) (end 147.4 63.6) (width 0.2) (layer "F.Cu") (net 4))
 (segment (start 146.199 63.901) (end 146.5 63.6) (width 0.2) (layer "F.Cu") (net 4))
 (segment (start 161.399 75.599) (end 151 65.2) (width 0.2) (layer "F.Cu") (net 4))
 (segment (start 144.525 100.03) (end 146.378 98.177) (width 0.2) (layer "F.Cu") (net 4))
 (segment (start 161.399 98.177) (end 161.399 75.599) (width 0.2) (layer "F.Cu") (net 4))
 (segment (start 146.486936 67.601) (end 146.199 67.313064) (width 0.2) (layer "F.Cu") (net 4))
 (segment (start 146.378 98.177) (end 161.399 98.177) (width 0.2) (layer "F.Cu") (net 4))
 (segment (start 159.621 96.2) (end 159.621 78.821) (width 0.2) (layer "F.Cu") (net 21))
 (segment (start 147.431661 79.023) (end 145.576 77.167339) (width 0.2) (layer "F.Cu") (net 21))
 (segment (start 145.576 76.734661) (end 136.442339 67.601) (width 0.2) (layer "F.Cu") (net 21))
 (segment (start 159.377 79.023) (end 147.431661 79.023) (width 0.2) (layer "F.Cu") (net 21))
 (segment (start 135.4 118) (end 139.6 118) (width 0.2) (layer "F.Cu") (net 21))
 (segment (start 135 118) (end 135.4 118) (width 0.2) (layer "F.Cu") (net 21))
 (segment (start 153.4 96.098) (end 153.502 96.2) (width 0.2) (layer "F.Cu") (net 21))
 (segment (start 129.285 100.03) (end 126.745 100.03) (width 0.2) (layer "F.Cu") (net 21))
 (segment (start 126.8 109.8) (end 135 118) (width 0.2) (layer "F.Cu") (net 21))
 (segment (start 159.621 78.821) (end 159.6 78.8) (width 0.2) (layer "F.Cu") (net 21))
 (segment (start 139.6 118) (end 153.4 104.2) (width 0.2) (layer "F.Cu") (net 21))
 (segment (start 159.6 78.8) (end 159.377 79.023) (width 0.2) (layer "F.Cu") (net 21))
 (segment (start 134.199 66.101) (end 134.5 65.8) (width 0.2) (layer "F.Cu") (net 21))
 (segment (start 134.199 67.313064) (end 134.199 66.101) (width 0.2) (layer "F.Cu") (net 21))
 (segment (start 153.502 96.2) (end 159.621 96.2) (width 0.2) (layer "F.Cu") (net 21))
 (segment (start 134.486936 67.601) (end 134.199 67.313064) (width 0.2) (layer "F.Cu") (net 21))
 (segment (start 134.5 65.8) (end 135.4 65.8) (width 0.2) (layer "F.Cu") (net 21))
 (segment (start 145.576 77.167339) (end 145.576 76.734661) (width 0.2) (layer "F.Cu") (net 21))
 (segment (start 136.442339 67.601) (end 134.486936 67.601) (width 0.2) (layer "F.Cu") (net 21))
 (via (at 126.8 109.8) (size 0.6) (drill 0.3) (layers "F.Cu" "B.Cu") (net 21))
 (via (at 153.4 104.2) (size 0.6) (drill 0.3) (layers "F.Cu" "B.Cu") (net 21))
 (via (at 153.4 96.098) (size 0.6) (drill 0.3) (layers "F.Cu" "B.Cu") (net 21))
 (segment (start 126.745 109.745) (end 126.8 109.8) (width 0.2) (layer "B.Cu") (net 21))
 (segment (start 153.4 104.2) (end 153.4 96.098) (width 0.2) (layer "B.Cu") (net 21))
 (segment (start 126.745 100.03) (end 126.745 109.745) (width 0.2) (layer "B.Cu") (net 21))
 (segment (start 120.35 118) (end 120.000308 118) (width 0.2) (layer "F.Cu") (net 28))
 (segment (start 120.000308 118) (end 114.998 112.997692) (width 0.2) (layer "F.Cu") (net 28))
 (segment (start 141.755 74.4) (end 144.525 77.17) (width 0.2) (layer "F.Cu") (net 28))
 (segment (start 114.998 75.8349) (end 116.4329 74.4) (width 0.2) (layer "F.Cu") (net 28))
 (segment (start 114.998 112.997692) (end 114.998 75.8349) (width 0.2) (layer "F.Cu") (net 28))
 (segment (start 116.4329 74.4) (end 141.755 74.4) (width 0.2) (layer "F.Cu") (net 28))
 (segment (start 160.022 78.221) (end 160.022 96.578) (width 0.2) (layer "F.Cu") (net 36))
 (segment (start 151.057 78.622) (end 158.8801 78.622) (width 0.2) (layer "F.Cu") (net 36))
 (segment (start 137.8 115.6) (end 137.4 116) (width 0.2) (layer "F.Cu") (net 36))
 (segment (start 158.8801 78.622) (end 159.2811 78.221) (width 0.2) (layer "F.Cu") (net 36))
 (segment (start 141.702 96.698) (end 140.8 97.6) (width 0.2) (layer "F.Cu") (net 36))
 (segment (start 160.022 96.578) (end 159.902 96.698) (width 0.2) (layer "F.Cu") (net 36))
 (segment (start 159.4 96.698) (end 141.702 96.698) (width 0.2) (layer "F.Cu") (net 36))
 (segment (start 159.902 96.698) (end 159.4 96.698) (width 0.2) (layer "F.Cu") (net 36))
 (segment (start 137.4 116) (end 135.4 116) (width 0.2) (layer "F.Cu") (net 36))
 (segment (start 159.2811 78.221) (end 160.022 78.221) (width 0.2) (layer "F.Cu") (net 36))
 (segment (start 149.605 77.17) (end 151.057 78.622) (width 0.2) (layer "F.Cu") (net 36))
 (via (at 137.8 115.6) (size 0.6) (drill 0.3) (layers "F.Cu" "B.Cu") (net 36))
 (via (at 140.8 97.6) (size 0.6) (drill 0.3) (layers "F.Cu" "B.Cu") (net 36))
 (segment (start 140.8 97.6) (end 140.8 102.701339) (width 0.2) (layer "B.Cu") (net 36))
 (segment (start 137.8 105.701339) (end 137.8 115.6) (width 0.2) (layer "B.Cu") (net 36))
 (segment (start 140.8 102.701339) (end 137.8 105.701339) (width 0.2) (layer "B.Cu") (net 36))
 (segment (start 115.8 111.6) (end 115.8 103) (width 0.2) (layer "F.Cu") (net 26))
 (segment (start 118.2 114) (end 115.8 111.6) (width 0.2) (layer "F.Cu") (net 26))
 (segment (start 131.6 102.4) (end 131.825 102.175) (width 0.2) (layer "F.Cu") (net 26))
 (segment (start 115.8 103) (end 116.4 102.4) (width 0.2) (layer "F.Cu") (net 26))
 (segment (start 120.35 114) (end 118.2 114) (width 0.2) (layer "F.Cu") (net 26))
 (segment (start 131.825 102.175) (end 131.825 100.03) (width 0.2) (layer "F.Cu") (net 26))
 (segment (start 116.4 102.4) (end 131.6 102.4) (width 0.2) (layer "F.Cu") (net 26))
 (segment (start 120.5 59.75) (end 120.5 67) (width 0.2) (layer "F.Cu") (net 24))
 (segment (start 118.4 120) (end 120.35 120) (width 0.2) (layer "F.Cu") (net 29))
 (segment (start 149.605 100.03) (end 150.656 98.979) (width 0.2) (layer "F.Cu") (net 29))
 (segment (start 117.4 121) (end 118.4 120) (width 0.2) (layer "F.Cu") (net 29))
 (segment (start 117.4 127.2) (end 117.4 121) (width 0.2) (layer "F.Cu") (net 29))
 (segment (start 160.200339 98.979) (end 164.601 103.379661) (width 0.2) (layer "F.Cu") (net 29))
 (segment (start 164.601 123.1661) (end 160.4301 127.337) (width 0.2) (layer "F.Cu") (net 29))
 (segment (start 164.601 103.379661) (end 164.601 123.1661) (width 0.2) (layer "F.Cu") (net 29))
 (segment (start 117.537 127.337) (end 117.4 127.2) (width 0.2) (layer "F.Cu") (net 29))
 (segment (start 160.4301 127.337) (end 117.537 127.337) (width 0.2) (layer "F.Cu") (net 29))
 (segment (start 150.656 98.979) (end 160.200339 98.979) (width 0.2) (layer "F.Cu") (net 29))
 (segment (start 145.3 97.5) (end 143.4 99.4) (width 0.2) (layer "F.Cu") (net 37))
 (segment (start 139 113.6) (end 138.6 114) (width 0.2) (layer "F.Cu") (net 37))
 (segment (start 160.200339 76.119) (end 160.824 76.742661) (width 0.2) (layer "F.Cu") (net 37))
 (segment (start 138.6 114) (end 135.4 114) (width 0.2) (layer "F.Cu") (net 37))
 (segment (start 160.7 97.5) (end 145.3 97.5) (width 0.2) (layer "F.Cu") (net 37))
 (segment (start 160.824 97.376) (end 160.7 97.5) (width 0.2) (layer "F.Cu") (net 37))
 (segment (start 147.065 77.17) (end 148.116 76.119) (width 0.2) (layer "F.Cu") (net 37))
 (segment (start 148.116 76.119) (end 160.200339 76.119) (width 0.2) (layer "F.Cu") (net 37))
 (segment (start 160.824 76.742661) (end 160.824 97.376) (width 0.2) (layer "F.Cu") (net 37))
 (via (at 139 113.6) (size 0.6) (drill 0.3) (layers "F.Cu" "B.Cu") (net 37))
 (via (at 143.4 99.4) (size 0.6) (drill 0.3) (layers "F.Cu" "B.Cu") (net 37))
 (segment (start 143.4 99.4) (end 143.4 109.2) (width 0.2) (layer "B.Cu") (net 37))
 (segment (start 143.4 109.2) (end 139 113.6) (width 0.2) (layer "B.Cu") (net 37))
 (segment (start 119.6329 116) (end 115.399 111.7661) (width 0.2) (layer "F.Cu") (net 27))
 (segment (start 120.35 116) (end 119.6329 116) (width 0.2) (layer "F.Cu") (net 27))
 (segment (start 116.6 74.8) (end 139.615 74.8) (width 0.2) (layer "F.Cu") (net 27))
 (segment (start 139.615 74.8) (end 141.985 77.17) (width 0.2) (layer "F.Cu") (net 27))
 (segment (start 115.399 111.7661) (end 115.399 76.001) (width 0.2) (layer "F.Cu") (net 27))
 (segment (start 115.399 76.001) (end 116.6 74.8) (width 0.2) (layer "F.Cu") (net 27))
 (segment (start 134.5 63.6) (end 135.4 63.6) (width 0.2) (layer "F.Cu") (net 19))
 (segment (start 133 65.6) (end 133 65.1) (width 0.2) (layer "F.Cu") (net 19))
 (segment (start 133 65.1) (end 134.5 63.6) (width 0.2) (layer "F.Cu") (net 19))
 (via (at 133 65.6) (size 0.6) (drill 0.3) (layers "F.Cu" "B.Cu") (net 19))
 (segment (start 126.745 77.17) (end 126.745 71.855) (width 0.2) (layer "B.Cu") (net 19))
 (segment (start 126.745 71.855) (end 133 65.6) (width 0.2) (layer "B.Cu") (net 19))
 (segment (start 116.48355 102.88355) (end 116.201 103.1661) (width 0.2) (layer "F.Cu") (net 30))
 (segment (start 134.365 100.03) (end 134.365 101.09066) (width 0.2) (layer "F.Cu") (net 30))
 (segment (start 122.126 113.426308) (end 122.126 121.699) (width 0.2) (layer "F.Cu") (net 30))
 (segment (start 116.201 103.1661) (end 116.201 111.4339) (width 0.2) (layer "F.Cu") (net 30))
 (segment (start 134.365 101.09066) (end 132.57211 102.88355) (width 0.2) (layer "F.Cu") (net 30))
 (segment (start 118.1671 113.4) (end 118.4 113.4) (width 0.2) (layer "F.Cu") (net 30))
 (segment (start 118.4 113.4) (end 118.736 113.064) (width 0.2) (layer "F.Cu") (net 30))
 (segment (start 121.825 122) (end 120.35 122) (width 0.2) (layer "F.Cu") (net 30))
 (segment (start 121.763692 113.064) (end 122.126 113.426308) (width 0.2) (layer "F.Cu") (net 30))
 (segment (start 132.57211 102.88355) (end 116.48355 102.88355) (width 0.2) (layer "F.Cu") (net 30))
 (segment (start 116.201 111.4339) (end 118.1671 113.4) (width 0.2) (layer "F.Cu") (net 30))
 (segment (start 118.736 113.064) (end 121.763692 113.064) (width 0.2) (layer "F.Cu") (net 30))
 (segment (start 122.126 121.699) (end 121.825 122) (width 0.2) (layer "F.Cu") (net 30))
 (segment (start 161.778 98.578) (end 161.8 98.6) (width 0.2) (layer "F.Cu") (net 3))
 (segment (start 148.517 98.578) (end 161.778 98.578) (width 0.2) (layer "F.Cu") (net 3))
 (segment (start 161.8 98.6) (end 161.8 75.4) (width 0.2) (layer "F.Cu") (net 3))
 (segment (start 151.1 64.7) (end 147.4 64.7) (width 0.2) (layer "F.Cu") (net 3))
 (segment (start 161.8 75.4) (end 151.1 64.7) (width 0.2) (layer "F.Cu") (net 3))
 (segment (start 147.065 100.03) (end 148.517 98.578) (width 0.2) (layer "F.Cu") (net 3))
 (segment (start 120.5 68.65) (end 120.5 74) (width 0.2) (layer "F.Cu") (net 23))
 (segment (start 120.5 74) (end 132.8 74) (width 0.2) (layer "F.Cu") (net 23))
 (segment (start 132.8 74) (end 133 73.8) (width 0.2) (layer "F.Cu") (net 23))
 (via (at 133 73.8) (size 0.6) (drill 0.3) (layers "F.Cu" "B.Cu") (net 23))
 (segment (start 134.365 75.165) (end 134.365 77.17) (width 0.2) (layer "B.Cu") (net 23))
 (segment (start 133 73.8) (end 134.365 75.165) (width 0.2) (layer "B.Cu") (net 23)))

